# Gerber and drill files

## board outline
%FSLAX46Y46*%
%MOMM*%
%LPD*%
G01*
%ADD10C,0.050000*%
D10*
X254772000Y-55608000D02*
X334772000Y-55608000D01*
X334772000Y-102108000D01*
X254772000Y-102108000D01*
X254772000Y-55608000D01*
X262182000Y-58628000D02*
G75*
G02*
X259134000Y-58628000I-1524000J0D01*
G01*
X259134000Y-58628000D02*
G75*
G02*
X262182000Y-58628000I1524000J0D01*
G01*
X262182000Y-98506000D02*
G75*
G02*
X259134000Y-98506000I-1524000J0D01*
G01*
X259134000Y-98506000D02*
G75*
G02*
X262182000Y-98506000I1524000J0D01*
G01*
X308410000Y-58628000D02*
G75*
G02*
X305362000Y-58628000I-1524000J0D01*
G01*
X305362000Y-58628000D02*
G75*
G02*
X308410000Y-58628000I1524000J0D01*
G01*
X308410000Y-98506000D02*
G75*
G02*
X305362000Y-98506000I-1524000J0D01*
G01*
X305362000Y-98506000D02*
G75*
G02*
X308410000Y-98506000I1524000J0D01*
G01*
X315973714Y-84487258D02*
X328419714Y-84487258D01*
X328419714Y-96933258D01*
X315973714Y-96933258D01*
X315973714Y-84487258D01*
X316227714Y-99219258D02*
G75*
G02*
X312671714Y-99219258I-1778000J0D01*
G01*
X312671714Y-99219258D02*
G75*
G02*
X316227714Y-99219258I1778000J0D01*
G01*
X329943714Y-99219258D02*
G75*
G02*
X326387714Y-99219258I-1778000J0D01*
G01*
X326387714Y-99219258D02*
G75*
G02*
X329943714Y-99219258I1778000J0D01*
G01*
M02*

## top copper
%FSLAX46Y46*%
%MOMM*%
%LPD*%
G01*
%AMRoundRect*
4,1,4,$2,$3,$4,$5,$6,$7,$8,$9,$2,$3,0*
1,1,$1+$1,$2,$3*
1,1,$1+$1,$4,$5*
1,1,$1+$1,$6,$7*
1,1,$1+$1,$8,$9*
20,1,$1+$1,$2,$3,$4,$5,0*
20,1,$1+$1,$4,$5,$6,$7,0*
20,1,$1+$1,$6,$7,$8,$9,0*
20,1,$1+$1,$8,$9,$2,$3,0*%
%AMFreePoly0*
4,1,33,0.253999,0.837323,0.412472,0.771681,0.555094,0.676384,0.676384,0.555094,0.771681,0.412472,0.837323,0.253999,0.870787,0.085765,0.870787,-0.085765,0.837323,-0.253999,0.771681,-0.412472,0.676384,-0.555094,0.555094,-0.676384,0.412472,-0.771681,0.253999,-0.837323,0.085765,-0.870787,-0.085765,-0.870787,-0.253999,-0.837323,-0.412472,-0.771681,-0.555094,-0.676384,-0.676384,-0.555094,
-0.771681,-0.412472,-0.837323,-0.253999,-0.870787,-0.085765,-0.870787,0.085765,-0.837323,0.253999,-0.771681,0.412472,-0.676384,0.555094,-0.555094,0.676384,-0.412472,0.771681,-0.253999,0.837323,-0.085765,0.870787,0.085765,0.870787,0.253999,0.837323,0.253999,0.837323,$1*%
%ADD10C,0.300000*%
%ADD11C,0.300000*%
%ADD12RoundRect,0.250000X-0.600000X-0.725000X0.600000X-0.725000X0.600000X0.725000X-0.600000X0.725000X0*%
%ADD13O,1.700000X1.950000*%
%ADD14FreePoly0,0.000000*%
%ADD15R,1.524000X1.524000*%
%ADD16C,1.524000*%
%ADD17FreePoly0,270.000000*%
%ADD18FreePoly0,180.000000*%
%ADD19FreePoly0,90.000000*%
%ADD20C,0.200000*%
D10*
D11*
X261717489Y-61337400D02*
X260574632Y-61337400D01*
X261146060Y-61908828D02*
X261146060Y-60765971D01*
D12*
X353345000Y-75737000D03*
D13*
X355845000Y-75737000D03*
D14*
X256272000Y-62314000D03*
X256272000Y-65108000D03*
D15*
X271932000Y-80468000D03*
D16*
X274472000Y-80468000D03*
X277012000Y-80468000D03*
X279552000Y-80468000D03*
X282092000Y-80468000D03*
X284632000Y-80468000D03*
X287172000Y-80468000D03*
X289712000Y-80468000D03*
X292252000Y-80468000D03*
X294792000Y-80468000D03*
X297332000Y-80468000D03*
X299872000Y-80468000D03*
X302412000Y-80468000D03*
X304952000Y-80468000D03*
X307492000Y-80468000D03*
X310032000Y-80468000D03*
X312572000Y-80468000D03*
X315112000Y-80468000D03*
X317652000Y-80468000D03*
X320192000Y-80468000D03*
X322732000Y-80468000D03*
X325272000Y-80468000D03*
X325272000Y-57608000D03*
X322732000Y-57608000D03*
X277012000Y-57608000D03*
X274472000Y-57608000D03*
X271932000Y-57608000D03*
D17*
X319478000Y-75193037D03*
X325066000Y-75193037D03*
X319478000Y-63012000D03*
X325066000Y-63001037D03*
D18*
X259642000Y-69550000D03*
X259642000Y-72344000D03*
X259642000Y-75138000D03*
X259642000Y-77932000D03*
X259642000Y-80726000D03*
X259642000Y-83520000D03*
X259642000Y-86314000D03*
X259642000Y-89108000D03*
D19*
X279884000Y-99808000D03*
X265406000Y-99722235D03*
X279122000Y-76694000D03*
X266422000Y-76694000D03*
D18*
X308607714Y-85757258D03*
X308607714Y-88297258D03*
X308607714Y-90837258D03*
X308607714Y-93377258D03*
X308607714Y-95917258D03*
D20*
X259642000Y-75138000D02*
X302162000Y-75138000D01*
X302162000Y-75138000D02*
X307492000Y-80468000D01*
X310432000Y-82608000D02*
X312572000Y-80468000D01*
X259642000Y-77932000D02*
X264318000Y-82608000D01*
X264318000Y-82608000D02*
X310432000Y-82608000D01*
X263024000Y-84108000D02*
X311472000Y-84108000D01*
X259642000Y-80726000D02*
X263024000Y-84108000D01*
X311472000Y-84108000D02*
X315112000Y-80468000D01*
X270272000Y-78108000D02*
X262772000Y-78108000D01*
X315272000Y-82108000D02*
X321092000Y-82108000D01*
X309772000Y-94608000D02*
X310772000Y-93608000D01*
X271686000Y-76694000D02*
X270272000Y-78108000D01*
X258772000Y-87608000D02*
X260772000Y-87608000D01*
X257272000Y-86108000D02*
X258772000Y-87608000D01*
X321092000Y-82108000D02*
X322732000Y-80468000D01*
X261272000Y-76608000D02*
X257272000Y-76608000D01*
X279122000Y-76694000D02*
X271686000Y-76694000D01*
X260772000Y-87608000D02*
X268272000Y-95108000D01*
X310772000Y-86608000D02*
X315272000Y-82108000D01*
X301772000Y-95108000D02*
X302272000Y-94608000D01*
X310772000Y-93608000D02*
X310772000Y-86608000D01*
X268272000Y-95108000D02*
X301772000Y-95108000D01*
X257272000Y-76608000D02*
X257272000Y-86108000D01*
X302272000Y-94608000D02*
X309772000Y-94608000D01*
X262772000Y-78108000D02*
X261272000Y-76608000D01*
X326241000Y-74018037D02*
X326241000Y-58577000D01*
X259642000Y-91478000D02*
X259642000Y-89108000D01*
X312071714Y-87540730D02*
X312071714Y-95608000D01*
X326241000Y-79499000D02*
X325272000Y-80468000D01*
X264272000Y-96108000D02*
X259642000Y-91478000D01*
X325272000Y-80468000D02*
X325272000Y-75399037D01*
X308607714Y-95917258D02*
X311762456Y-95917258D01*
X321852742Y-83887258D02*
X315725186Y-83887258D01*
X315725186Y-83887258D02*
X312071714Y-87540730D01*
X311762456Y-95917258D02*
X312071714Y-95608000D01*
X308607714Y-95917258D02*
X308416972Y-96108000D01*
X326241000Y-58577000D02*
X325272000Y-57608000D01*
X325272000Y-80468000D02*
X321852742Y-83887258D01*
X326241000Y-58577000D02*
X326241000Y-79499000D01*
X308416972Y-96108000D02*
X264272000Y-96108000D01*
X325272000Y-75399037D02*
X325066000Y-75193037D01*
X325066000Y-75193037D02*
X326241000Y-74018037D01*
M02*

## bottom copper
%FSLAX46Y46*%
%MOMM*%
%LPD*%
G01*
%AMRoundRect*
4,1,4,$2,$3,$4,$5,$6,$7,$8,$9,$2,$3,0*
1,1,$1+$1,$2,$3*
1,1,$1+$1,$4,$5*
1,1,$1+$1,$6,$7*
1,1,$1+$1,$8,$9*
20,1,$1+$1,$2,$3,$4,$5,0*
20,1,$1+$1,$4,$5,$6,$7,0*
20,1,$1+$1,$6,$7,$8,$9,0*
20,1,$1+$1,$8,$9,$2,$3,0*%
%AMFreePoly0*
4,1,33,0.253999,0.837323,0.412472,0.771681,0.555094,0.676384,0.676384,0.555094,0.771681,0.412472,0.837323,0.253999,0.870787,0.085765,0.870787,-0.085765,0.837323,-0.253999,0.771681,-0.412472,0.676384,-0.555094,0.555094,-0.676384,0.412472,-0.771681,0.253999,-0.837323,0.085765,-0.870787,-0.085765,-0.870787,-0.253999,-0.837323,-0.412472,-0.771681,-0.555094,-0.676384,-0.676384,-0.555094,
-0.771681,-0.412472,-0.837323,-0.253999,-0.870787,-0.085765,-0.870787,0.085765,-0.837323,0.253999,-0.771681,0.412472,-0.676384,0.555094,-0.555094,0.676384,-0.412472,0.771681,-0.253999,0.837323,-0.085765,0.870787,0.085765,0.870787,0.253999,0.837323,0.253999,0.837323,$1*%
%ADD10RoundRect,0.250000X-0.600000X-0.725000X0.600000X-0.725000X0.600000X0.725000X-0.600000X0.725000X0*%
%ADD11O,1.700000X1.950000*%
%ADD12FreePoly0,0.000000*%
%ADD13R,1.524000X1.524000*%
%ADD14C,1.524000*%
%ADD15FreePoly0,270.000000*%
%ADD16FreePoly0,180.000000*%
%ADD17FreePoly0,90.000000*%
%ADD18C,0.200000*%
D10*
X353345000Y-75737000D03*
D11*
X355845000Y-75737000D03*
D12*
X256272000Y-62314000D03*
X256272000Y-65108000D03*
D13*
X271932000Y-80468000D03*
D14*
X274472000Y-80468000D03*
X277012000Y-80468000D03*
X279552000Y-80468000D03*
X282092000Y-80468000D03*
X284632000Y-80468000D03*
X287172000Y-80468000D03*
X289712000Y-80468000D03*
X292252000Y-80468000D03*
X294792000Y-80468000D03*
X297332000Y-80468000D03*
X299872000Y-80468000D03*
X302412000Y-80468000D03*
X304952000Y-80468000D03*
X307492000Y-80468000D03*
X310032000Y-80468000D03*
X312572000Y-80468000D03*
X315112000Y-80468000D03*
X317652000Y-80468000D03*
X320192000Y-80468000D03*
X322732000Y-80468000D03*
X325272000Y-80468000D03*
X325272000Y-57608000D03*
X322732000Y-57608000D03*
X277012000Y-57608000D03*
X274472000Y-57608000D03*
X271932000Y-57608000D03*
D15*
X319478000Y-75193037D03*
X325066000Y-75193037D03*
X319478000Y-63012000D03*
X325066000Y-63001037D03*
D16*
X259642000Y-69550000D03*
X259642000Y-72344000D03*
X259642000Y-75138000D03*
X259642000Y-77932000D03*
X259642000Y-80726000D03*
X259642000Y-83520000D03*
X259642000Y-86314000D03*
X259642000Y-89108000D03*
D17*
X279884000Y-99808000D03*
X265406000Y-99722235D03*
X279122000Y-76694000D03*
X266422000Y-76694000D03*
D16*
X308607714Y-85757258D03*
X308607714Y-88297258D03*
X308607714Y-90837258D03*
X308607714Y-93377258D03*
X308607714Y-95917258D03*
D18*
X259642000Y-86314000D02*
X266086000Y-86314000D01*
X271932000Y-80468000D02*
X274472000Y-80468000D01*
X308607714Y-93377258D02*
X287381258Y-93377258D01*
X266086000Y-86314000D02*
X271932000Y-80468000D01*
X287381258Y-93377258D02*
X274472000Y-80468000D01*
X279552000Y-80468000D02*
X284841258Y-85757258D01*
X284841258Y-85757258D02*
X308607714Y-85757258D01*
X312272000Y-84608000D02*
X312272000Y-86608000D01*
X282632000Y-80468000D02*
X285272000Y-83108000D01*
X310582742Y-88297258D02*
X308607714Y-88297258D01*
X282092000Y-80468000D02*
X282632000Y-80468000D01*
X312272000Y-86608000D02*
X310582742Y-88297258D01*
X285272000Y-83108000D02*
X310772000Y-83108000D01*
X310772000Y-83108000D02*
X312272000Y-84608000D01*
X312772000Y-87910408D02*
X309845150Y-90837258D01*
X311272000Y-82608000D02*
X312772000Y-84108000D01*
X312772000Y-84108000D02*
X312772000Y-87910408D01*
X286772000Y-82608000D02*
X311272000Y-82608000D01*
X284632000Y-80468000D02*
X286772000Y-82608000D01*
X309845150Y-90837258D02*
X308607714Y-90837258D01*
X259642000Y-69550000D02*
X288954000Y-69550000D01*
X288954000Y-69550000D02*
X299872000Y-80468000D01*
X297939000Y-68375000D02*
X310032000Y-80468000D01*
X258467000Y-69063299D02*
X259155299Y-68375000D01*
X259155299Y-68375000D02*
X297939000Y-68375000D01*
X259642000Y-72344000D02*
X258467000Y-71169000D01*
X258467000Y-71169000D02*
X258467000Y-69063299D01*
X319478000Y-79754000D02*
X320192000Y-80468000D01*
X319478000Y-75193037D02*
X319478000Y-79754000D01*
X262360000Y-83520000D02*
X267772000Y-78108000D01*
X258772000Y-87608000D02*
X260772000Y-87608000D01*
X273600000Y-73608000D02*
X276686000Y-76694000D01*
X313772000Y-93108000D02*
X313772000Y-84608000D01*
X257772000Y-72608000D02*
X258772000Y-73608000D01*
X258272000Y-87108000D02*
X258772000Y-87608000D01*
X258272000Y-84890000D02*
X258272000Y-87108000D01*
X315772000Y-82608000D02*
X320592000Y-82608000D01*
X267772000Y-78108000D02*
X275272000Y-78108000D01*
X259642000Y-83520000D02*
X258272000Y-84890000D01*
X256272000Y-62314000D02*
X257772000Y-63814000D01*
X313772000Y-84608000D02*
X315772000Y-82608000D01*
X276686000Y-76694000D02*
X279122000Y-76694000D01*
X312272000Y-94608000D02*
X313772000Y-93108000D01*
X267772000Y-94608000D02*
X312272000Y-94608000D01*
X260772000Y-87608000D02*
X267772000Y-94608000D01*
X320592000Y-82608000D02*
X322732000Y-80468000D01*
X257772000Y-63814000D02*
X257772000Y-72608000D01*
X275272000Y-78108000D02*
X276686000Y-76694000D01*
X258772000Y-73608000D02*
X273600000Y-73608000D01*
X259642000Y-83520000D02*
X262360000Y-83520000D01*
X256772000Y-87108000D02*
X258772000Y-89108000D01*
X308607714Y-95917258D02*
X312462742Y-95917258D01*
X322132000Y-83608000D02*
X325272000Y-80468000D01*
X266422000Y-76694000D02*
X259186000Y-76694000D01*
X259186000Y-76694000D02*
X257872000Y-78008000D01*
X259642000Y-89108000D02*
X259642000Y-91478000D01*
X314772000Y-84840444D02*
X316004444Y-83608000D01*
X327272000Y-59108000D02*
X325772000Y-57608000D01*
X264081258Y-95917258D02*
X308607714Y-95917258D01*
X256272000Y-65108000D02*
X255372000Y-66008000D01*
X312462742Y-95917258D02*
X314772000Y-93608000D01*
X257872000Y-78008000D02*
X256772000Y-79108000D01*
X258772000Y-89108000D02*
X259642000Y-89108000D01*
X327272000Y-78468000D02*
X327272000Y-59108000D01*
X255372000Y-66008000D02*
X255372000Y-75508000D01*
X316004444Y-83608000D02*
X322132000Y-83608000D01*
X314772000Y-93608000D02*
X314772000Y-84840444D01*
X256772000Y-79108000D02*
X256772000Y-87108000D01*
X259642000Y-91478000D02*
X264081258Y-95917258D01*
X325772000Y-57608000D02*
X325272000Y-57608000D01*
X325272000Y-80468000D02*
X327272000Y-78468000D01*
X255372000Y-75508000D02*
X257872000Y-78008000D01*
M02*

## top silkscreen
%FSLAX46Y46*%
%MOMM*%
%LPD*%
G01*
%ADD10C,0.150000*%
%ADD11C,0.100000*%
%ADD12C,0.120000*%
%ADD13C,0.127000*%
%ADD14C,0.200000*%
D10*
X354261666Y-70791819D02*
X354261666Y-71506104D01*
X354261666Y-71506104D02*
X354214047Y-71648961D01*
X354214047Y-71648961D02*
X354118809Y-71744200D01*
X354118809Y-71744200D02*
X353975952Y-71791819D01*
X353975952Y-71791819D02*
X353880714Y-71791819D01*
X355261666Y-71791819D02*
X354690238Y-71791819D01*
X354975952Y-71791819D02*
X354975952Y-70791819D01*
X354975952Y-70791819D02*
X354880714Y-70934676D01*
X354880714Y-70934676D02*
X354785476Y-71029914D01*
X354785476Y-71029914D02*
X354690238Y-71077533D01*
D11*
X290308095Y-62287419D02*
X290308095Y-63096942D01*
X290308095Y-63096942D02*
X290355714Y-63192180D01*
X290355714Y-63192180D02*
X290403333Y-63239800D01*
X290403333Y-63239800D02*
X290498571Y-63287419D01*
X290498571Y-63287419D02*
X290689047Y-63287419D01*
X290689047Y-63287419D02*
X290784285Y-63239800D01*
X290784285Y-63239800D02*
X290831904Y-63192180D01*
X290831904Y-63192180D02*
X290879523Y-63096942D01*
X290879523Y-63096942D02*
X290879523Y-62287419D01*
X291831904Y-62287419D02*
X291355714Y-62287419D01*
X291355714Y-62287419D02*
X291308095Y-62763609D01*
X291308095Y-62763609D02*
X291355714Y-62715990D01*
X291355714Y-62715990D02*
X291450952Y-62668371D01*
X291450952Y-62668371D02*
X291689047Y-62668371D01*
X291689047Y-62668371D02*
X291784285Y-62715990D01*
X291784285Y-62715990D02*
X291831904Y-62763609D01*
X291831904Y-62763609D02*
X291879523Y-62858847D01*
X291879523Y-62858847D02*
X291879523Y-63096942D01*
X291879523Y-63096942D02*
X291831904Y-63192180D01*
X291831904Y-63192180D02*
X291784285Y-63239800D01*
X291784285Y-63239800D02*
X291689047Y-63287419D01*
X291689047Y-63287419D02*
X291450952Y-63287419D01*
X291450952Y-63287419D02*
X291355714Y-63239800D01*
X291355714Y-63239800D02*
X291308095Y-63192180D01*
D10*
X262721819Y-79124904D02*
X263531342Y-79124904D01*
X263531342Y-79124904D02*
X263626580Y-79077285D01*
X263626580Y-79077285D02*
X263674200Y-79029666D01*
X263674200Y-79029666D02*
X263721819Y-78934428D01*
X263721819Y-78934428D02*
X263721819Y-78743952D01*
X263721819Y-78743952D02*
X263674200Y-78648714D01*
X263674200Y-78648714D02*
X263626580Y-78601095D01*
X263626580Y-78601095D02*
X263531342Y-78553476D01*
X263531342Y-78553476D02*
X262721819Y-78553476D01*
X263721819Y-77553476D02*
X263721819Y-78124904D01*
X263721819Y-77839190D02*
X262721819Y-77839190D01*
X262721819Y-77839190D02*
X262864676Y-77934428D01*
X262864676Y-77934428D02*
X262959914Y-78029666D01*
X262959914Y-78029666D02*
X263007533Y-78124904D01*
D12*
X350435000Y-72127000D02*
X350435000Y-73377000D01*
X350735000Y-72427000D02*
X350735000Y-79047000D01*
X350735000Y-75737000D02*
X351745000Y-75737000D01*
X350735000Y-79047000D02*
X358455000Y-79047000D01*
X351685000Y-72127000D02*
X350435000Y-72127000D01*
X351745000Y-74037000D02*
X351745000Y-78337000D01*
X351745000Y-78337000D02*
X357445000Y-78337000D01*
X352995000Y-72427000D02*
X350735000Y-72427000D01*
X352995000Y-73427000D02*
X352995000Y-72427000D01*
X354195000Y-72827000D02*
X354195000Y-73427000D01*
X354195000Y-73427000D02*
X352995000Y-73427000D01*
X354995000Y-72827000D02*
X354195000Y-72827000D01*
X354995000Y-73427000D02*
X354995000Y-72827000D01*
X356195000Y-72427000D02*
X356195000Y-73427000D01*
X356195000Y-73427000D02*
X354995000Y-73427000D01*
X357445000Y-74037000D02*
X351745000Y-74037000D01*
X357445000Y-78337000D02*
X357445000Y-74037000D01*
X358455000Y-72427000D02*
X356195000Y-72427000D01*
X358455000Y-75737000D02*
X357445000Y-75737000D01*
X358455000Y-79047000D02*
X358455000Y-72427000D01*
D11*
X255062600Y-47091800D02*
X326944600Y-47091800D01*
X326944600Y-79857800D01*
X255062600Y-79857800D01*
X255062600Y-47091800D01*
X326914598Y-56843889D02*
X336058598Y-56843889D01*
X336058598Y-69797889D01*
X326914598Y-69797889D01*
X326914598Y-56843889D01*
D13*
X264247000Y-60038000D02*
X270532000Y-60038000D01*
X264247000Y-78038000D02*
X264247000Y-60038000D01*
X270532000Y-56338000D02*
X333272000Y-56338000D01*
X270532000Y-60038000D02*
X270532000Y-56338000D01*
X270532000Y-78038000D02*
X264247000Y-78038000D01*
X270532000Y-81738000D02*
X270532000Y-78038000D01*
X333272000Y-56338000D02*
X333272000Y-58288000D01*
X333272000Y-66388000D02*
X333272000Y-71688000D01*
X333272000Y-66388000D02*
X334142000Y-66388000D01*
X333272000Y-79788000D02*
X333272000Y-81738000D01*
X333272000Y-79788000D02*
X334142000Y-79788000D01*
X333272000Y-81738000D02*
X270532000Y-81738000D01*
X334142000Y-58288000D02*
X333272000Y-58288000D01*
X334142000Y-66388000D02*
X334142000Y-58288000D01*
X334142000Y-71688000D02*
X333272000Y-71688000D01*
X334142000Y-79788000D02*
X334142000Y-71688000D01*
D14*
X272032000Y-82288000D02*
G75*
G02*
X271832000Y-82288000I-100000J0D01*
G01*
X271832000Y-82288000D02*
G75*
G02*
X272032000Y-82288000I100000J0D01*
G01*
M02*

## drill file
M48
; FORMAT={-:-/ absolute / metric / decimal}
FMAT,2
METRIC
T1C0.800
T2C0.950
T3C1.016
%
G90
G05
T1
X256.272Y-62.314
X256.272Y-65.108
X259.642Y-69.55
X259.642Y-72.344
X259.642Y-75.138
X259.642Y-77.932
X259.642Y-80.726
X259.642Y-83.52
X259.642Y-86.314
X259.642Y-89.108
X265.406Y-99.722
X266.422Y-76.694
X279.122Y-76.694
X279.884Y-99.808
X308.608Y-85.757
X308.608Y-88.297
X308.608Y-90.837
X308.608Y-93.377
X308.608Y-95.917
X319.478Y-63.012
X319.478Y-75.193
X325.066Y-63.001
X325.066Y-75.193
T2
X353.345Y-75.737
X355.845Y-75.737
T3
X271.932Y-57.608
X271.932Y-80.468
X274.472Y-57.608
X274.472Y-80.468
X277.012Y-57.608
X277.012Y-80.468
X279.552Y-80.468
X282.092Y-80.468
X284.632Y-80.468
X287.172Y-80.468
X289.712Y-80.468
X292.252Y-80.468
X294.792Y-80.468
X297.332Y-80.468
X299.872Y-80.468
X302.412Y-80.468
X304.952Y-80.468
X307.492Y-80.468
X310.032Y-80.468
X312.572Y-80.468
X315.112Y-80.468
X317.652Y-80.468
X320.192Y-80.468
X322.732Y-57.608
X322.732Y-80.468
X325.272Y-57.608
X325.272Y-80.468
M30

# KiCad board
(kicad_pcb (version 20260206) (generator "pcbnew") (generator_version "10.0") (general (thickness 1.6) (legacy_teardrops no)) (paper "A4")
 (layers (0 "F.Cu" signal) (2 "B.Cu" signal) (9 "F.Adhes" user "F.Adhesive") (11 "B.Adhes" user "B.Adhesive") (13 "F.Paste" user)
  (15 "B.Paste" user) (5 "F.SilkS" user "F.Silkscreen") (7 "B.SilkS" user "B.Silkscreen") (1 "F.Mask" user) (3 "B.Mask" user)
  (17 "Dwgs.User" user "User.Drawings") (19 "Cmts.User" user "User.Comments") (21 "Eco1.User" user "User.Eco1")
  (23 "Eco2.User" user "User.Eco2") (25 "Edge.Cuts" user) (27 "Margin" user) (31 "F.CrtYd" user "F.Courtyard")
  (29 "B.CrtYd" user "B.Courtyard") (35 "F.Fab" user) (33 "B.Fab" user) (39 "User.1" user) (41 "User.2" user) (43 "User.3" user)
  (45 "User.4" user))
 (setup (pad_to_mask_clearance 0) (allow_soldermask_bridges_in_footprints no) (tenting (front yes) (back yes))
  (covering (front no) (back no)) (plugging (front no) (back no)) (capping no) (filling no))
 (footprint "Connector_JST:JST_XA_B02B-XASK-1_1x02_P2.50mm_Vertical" (layer "F.Cu") (at 353.345 75.737)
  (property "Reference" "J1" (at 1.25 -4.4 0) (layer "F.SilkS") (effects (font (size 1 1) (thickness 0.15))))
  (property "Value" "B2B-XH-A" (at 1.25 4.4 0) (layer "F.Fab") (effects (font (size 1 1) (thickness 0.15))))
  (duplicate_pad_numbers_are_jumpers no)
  (fp_line (start -2.91 -3.61) (end -2.91 -2.36) (stroke (width 0.12) (type solid)) (layer "F.SilkS"))
  (fp_line (start -2.61 -3.31) (end -2.61 3.31) (stroke (width 0.12) (type solid)) (layer "F.SilkS"))
  (fp_line (start -2.61 0) (end -1.6 0) (stroke (width 0.12) (type solid)) (layer "F.SilkS"))
  (fp_line (start -2.61 3.31) (end 5.11 3.31) (stroke (width 0.12) (type solid)) (layer "F.SilkS"))
  (fp_line (start -1.66 -3.61) (end -2.91 -3.61) (stroke (width 0.12) (type solid)) (layer "F.SilkS"))
  (fp_line (start -1.6 -1.7) (end -1.6 2.6) (stroke (width 0.12) (type solid)) (layer "F.SilkS"))
  (fp_line (start -1.6 2.6) (end 4.1 2.6) (stroke (width 0.12) (type solid)) (layer "F.SilkS"))
  (fp_line (start -0.35 -3.31) (end -2.61 -3.31) (stroke (width 0.12) (type solid)) (layer "F.SilkS"))
  (fp_line (start -0.35 -2.31) (end -0.35 -3.31) (stroke (width 0.12) (type solid)) (layer "F.SilkS"))
  (fp_line (start 0.85 -2.91) (end 0.85 -2.31) (stroke (width 0.12) (type solid)) (layer "F.SilkS"))
  (fp_line (start 0.85 -2.31) (end -0.35 -2.31) (stroke (width 0.12) (type solid)) (layer "F.SilkS"))
  (fp_line (start 1.65 -2.91) (end 0.85 -2.91) (stroke (width 0.12) (type solid)) (layer "F.SilkS"))
  (fp_line (start 1.65 -2.31) (end 1.65 -2.91) (stroke (width 0.12) (type solid)) (layer "F.SilkS"))
  (fp_line (start 2.85 -3.31) (end 2.85 -2.31) (stroke (width 0.12) (type solid)) (layer "F.SilkS"))
  (fp_line (start 2.85 -2.31) (end 1.65 -2.31) (stroke (width 0.12) (type solid)) (layer "F.SilkS"))
  (fp_line (start 4.1 -1.7) (end -1.6 -1.7) (stroke (width 0.12) (type solid)) (layer "F.SilkS"))
  (fp_line (start 4.1 2.6) (end 4.1 -1.7) (stroke (width 0.12) (type solid)) (layer "F.SilkS"))
  (fp_line (start 5.11 -3.31) (end 2.85 -3.31) (stroke (width 0.12) (type solid)) (layer "F.SilkS"))
  (fp_line (start 5.11 0) (end 4.1 0) (stroke (width 0.12) (type solid)) (layer "F.SilkS"))
  (fp_line (start 5.11 3.31) (end 5.11 -3.31) (stroke (width 0.12) (type solid)) (layer "F.SilkS"))
  (pad "1" thru_hole roundrect (at 0 0) (size 1.7 1.95) (drill 0.95) (layers "*.Cu" "*.Mask") (remove_unused_layers no)
   (roundrect_rratio 0.147059) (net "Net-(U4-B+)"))
  (pad "2" thru_hole oval (at 2.5 0) (size 1.7 1.95) (drill 0.95) (layers "*.Cu" "*.Mask") (remove_unused_layers no) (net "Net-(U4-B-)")))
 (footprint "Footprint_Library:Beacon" (layer "F.Cu") (at 291.07 63.33)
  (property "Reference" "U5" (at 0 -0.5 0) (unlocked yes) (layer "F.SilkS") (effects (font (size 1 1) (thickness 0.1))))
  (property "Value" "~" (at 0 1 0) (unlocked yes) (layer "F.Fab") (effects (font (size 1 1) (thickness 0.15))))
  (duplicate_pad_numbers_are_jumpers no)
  (fp_rect (start -36.0074 -16.2382) (end 35.8746 16.5278) (stroke (width 0.1) (type default)) (fill no) (layer "F.SilkS"))
  (fp_rect (start 35.844598 -6.486111) (end 44.988598 6.467889) (stroke (width 0.1) (type default)) (fill no) (layer "F.SilkS"))
  (pad "1" thru_hole custom (at -34.798 -1.016) (size 1.75 1.75) (drill 0.8) (layers "*.Cu" "*.Mask") (remove_unused_layers no)
   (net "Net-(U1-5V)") (thermal_bridge_angle 90) (options (clearance outline) (anchor circle)) (primitives))
  (pad "2" thru_hole custom (at -34.798 1.778) (size 1.75 1.75) (drill 0.8) (layers "*.Cu" "*.Mask") (remove_unused_layers no)
   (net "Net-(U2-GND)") (thermal_bridge_angle 90) (options (clearance outline) (anchor circle)) (primitives)))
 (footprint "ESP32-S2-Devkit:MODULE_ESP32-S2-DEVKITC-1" (layer "F.Cu") (at 301.902 69.038 90)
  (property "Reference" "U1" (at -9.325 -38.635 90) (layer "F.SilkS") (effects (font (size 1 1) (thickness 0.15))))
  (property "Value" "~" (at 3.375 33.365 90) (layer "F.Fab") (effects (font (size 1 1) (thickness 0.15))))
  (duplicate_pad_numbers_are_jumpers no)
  (fp_line (start 9 -37.655) (end 9 -31.37) (stroke (width 0.127) (type solid)) (layer "F.SilkS"))
  (fp_line (start -9 -37.655) (end 9 -37.655) (stroke (width 0.127) (type solid)) (layer "F.SilkS"))
  (fp_line (start 12.7 -31.37) (end 12.7 31.37) (stroke (width 0.127) (type solid)) (layer "F.SilkS"))
  (fp_line (start 9 -31.37) (end 12.7 -31.37) (stroke (width 0.127) (type solid)) (layer "F.SilkS"))
  (fp_line (start -9 -31.37) (end -9 -37.655) (stroke (width 0.127) (type solid)) (layer "F.SilkS"))
  (fp_line (start -12.7 -31.37) (end -9 -31.37) (stroke (width 0.127) (type solid)) (layer "F.SilkS"))
  (fp_line (start 12.7 31.37) (end 10.75 31.37) (stroke (width 0.127) (type solid)) (layer "F.SilkS"))
  (fp_line (start 2.65 31.37) (end -2.65 31.37) (stroke (width 0.127) (type solid)) (layer "F.SilkS"))
  (fp_line (start 2.65 31.37) (end 2.65 32.24) (stroke (width 0.127) (type solid)) (layer "F.SilkS"))
  (fp_line (start -10.75 31.37) (end -12.7 31.37) (stroke (width 0.127) (type solid)) (layer "F.SilkS"))
  (fp_line (start -10.75 31.37) (end -10.75 32.24) (stroke (width 0.127) (type solid)) (layer "F.SilkS"))
  (fp_line (start -12.7 31.37) (end -12.7 -31.37) (stroke (width 0.127) (type solid)) (layer "F.SilkS"))
  (fp_line (start 10.75 32.24) (end 10.75 31.37) (stroke (width 0.127) (type solid)) (layer "F.SilkS"))
  (fp_line (start 2.65 32.24) (end 10.75 32.24) (stroke (width 0.127) (type solid)) (layer "F.SilkS"))
  (fp_line (start -2.65 32.24) (end -2.65 31.37) (stroke (width 0.127) (type solid)) (layer "F.SilkS"))
  (fp_line (start -10.75 32.24) (end -2.65 32.24) (stroke (width 0.127) (type solid)) (layer "F.SilkS"))
  (fp_circle (center -13.25 -29.97) (end -13.15 -29.97) (stroke (width 0.2) (type solid)) (fill no) (layer "F.SilkS"))
  (pad "1" thru_hole rect (at -11.43 -29.97 90) (size 1.524 1.524) (drill 1.016) (layers "*.Cu" "*.Mask") (remove_unused_layers no)
   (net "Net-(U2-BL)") (solder_mask_margin 0.102))
  (pad "2" thru_hole circle (at -11.43 -27.43 90) (size 1.524 1.524) (drill 1.016) (layers "*.Cu" "*.Mask") (remove_unused_layers no)
   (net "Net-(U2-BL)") (solder_mask_margin 0.102))
  (pad "3" thru_hole circle (at -11.43 -24.89 90) (size 1.524 1.524) (drill 1.016) (layers "*.Cu" "*.Mask") (remove_unused_layers no)
   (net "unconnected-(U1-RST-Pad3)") (solder_mask_margin 0.102))
  (pad "4" thru_hole circle (at -11.43 -22.35 90) (size 1.524 1.524) (drill 1.016) (layers "*.Cu" "*.Mask") (remove_unused_layers no)
   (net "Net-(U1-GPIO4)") (solder_mask_margin 0.102))
  (pad "5" thru_hole circle (at -11.43 -19.81 90) (size 1.524 1.524) (drill 1.016) (layers "*.Cu" "*.Mask") (remove_unused_layers no)
   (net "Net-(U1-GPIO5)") (solder_mask_margin 0.102))
  (pad "6" thru_hole circle (at -11.43 -17.27 90) (size 1.524 1.524) (drill 1.016) (layers "*.Cu" "*.Mask") (remove_unused_layers no)
   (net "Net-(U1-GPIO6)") (solder_mask_margin 0.102))
  (pad "7" thru_hole circle (at -11.43 -14.73 90) (size 1.524 1.524) (drill 1.016) (layers "*.Cu" "*.Mask") (remove_unused_layers no)
   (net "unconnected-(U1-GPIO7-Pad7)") (solder_mask_margin 0.102))
  (pad "8" thru_hole circle (at -11.43 -12.19 90) (size 1.524 1.524) (drill 1.016) (layers "*.Cu" "*.Mask") (remove_unused_layers no)
   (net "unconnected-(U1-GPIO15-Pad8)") (solder_mask_margin 0.102))
  (pad "9" thru_hole circle (at -11.43 -9.65 90) (size 1.524 1.524) (drill 1.016) (layers "*.Cu" "*.Mask") (remove_unused_layers no)
   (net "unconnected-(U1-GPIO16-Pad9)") (solder_mask_margin 0.102))
  (pad "10" thru_hole circle (at -11.43 -7.11 90) (size 1.524 1.524) (drill 1.016) (layers "*.Cu" "*.Mask") (remove_unused_layers no)
   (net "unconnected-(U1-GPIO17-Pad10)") (solder_mask_margin 0.102))
  (pad "11" thru_hole circle (at -11.43 -4.57 90) (size 1.524 1.524) (drill 1.016) (layers "*.Cu" "*.Mask") (remove_unused_layers no)
   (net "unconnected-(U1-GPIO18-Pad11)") (solder_mask_margin 0.102))
  (pad "12" thru_hole circle (at -11.43 -2.03 90) (size 1.524 1.524) (drill 1.016) (layers "*.Cu" "*.Mask") (remove_unused_layers no)
   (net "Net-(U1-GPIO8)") (solder_mask_margin 0.102))
  (pad "13" thru_hole circle (at -11.43 0.51 90) (size 1.524 1.524) (drill 1.016) (layers "*.Cu" "*.Mask") (remove_unused_layers no)
   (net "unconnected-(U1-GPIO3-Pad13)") (solder_mask_margin 0.102))
  (pad "14" thru_hole circle (at -11.43 3.05 90) (size 1.524 1.524) (drill 1.016) (layers "*.Cu" "*.Mask") (remove_unused_layers no)
   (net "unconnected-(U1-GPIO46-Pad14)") (solder_mask_margin 0.102))
  (pad "15" thru_hole circle (at -11.43 5.59 90) (size 1.524 1.524) (drill 1.016) (layers "*.Cu" "*.Mask") (remove_unused_layers no)
   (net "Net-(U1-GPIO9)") (solder_mask_margin 0.102))
  (pad "16" thru_hole circle (at -11.43 8.13 90) (size 1.524 1.524) (drill 1.016) (layers "*.Cu" "*.Mask") (remove_unused_layers no)
   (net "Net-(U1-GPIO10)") (solder_mask_margin 0.102))
  (pad "17" thru_hole circle (at -11.43 10.67 90) (size 1.524 1.524) (drill 1.016) (layers "*.Cu" "*.Mask") (remove_unused_layers no)
   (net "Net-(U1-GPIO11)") (solder_mask_margin 0.102))
  (pad "18" thru_hole circle (at -11.43 13.21 90) (size 1.524 1.524) (drill 1.016) (layers "*.Cu" "*.Mask") (remove_unused_layers no)
   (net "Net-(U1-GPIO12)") (solder_mask_margin 0.102))
  (pad "19" thru_hole circle (at -11.43 15.75 90) (size 1.524 1.524) (drill 1.016) (layers "*.Cu" "*.Mask") (remove_unused_layers no)
   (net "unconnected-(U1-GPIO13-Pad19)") (solder_mask_margin 0.102))
  (pad "20" thru_hole circle (at -11.43 18.29 90) (size 1.524 1.524) (drill 1.016) (layers "*.Cu" "*.Mask") (remove_unused_layers no)
   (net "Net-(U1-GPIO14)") (solder_mask_margin 0.102))
  (pad "21" thru_hole circle (at -11.43 20.83 90) (size 1.524 1.524) (drill 1.016) (layers "*.Cu" "*.Mask") (remove_unused_layers no)
   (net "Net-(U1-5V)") (solder_mask_margin 0.102))
  (pad "22" thru_hole circle (at -11.43 23.37 90) (size 1.524 1.524) (drill 1.016) (layers "*.Cu" "*.Mask") (remove_unused_layers no)
   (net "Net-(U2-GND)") (solder_mask_margin 0.102))
  (pad "23" thru_hole circle (at 11.43 23.37 90) (size 1.524 1.524) (drill 1.016) (layers "*.Cu" "*.Mask") (remove_unused_layers no)
   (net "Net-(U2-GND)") (solder_mask_margin 0.102))
  (pad "24" thru_hole circle (at 11.43 20.83 90) (size 1.524 1.524) (drill 1.016) (layers "*.Cu" "*.Mask") (remove_unused_layers no)
   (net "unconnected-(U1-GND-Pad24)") (solder_mask_margin 0.102))
  (pad "42" thru_hole circle (at 11.43 -24.89 90) (size 1.524 1.524) (drill 1.016) (layers "*.Cu" "*.Mask") (remove_unused_layers no)
   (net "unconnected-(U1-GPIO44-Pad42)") (solder_mask_margin 0.102))
  (pad "43" thru_hole circle (at 11.43 -27.43 90) (size 1.524 1.524) (drill 1.016) (layers "*.Cu" "*.Mask") (remove_unused_layers no)
   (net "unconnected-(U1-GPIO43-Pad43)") (solder_mask_margin 0.102))
  (pad "44" thru_hole circle (at 11.43 -29.97 90) (size 1.524 1.524) (drill 1.016) (layers "*.Cu" "*.Mask") (remove_unused_layers no)
   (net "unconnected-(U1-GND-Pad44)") (solder_mask_margin 0.102)))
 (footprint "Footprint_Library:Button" (layer "B.Cu") (at 322.272 69.108 -90)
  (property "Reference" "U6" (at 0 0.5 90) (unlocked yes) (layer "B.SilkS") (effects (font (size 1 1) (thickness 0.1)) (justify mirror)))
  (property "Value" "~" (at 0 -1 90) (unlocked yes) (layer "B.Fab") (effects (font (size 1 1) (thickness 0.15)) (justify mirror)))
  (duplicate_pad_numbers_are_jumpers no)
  (pad "1" thru_hole custom (at 6.085037 2.794 270) (size 1.75 1.75) (drill 0.8) (layers "*.Cu" "*.Mask") (remove_unused_layers no)
   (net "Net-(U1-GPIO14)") (thermal_bridge_angle 90) (options (clearance outline) (anchor circle)) (primitives))
  (pad "2" thru_hole custom (at 6.085037 -2.794 270) (size 1.75 1.75) (drill 0.8) (layers "*.Cu" "*.Mask") (remove_unused_layers no)
   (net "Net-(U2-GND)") (thermal_bridge_angle 90) (options (clearance outline) (anchor circle)) (primitives))
  (pad "3" thru_hole custom (at -6.096 2.794 270) (size 1.75 1.75) (drill 0.8) (layers "*.Cu" "*.Mask") (remove_unused_layers no)
   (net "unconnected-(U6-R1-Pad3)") (thermal_bridge_angle 90) (options (clearance outline) (anchor circle)) (primitives))
  (pad "4" thru_hole custom (at -6.106963 -2.794 270) (size 1.75 1.75) (drill 0.8) (layers "*.Cu" "*.Mask") (remove_unused_layers no)
   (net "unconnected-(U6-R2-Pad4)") (thermal_bridge_angle 90) (options (clearance outline) (anchor circle)) (primitives)))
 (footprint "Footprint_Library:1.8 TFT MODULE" (layer "B.Cu") (at 283.772 80.218 180)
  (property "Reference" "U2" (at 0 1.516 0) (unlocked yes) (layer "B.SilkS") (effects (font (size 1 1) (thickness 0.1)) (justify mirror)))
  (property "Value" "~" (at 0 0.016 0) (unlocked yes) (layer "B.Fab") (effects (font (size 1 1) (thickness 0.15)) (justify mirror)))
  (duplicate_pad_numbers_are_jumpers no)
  (fp_circle (center 23.114 21.59) (end 24.638 21.59) (stroke (width 0.05) (type default)) (fill no) (layer "Edge.Cuts"))
  (fp_circle (center 23.114 -18.288) (end 24.638 -18.288) (stroke (width 0.05) (type default)) (fill no) (layer "Edge.Cuts"))
  (fp_circle (center -23.114 21.59) (end -21.59 21.59) (stroke (width 0.05) (type default)) (fill no) (layer "Edge.Cuts"))
  (fp_circle (center -23.114 -18.288) (end -21.59 -18.288) (stroke (width 0.05) (type default)) (fill no) (layer "Edge.Cuts"))
  (pad "1" thru_hole custom (at 24.13 10.668 180) (size 1.75 1.75) (drill 0.8) (layers "*.Cu" "*.Mask") (remove_unused_layers no)
   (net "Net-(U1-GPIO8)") (thermal_bridge_angle 90) (options (clearance outline) (anchor circle)) (primitives))
  (pad "2" thru_hole custom (at 24.13 7.874 180) (size 1.75 1.75) (drill 0.8) (layers "*.Cu" "*.Mask") (remove_unused_layers no)
   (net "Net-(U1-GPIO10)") (thermal_bridge_angle 90) (options (clearance outline) (anchor circle)) (primitives))
  (pad "3" thru_hole custom (at 24.13 5.08 180) (size 1.75 1.75) (drill 0.8) (layers "*.Cu" "*.Mask") (remove_unused_layers no)
   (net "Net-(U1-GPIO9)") (thermal_bridge_angle 90) (options (clearance outline) (anchor circle)) (primitives))
  (pad "4" thru_hole custom (at 24.13 2.286 180) (size 1.75 1.75) (drill 0.8) (layers "*.Cu" "*.Mask") (remove_unused_layers no)
   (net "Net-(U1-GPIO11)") (thermal_bridge_angle 90) (options (clearance outline) (anchor circle)) (primitives))
  (pad "5" thru_hole custom (at 24.13 -0.508 180) (size 1.75 1.75) (drill 0.8) (layers "*.Cu" "*.Mask") (remove_unused_layers no)
   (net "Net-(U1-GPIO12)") (thermal_bridge_angle 90) (options (clearance outline) (anchor circle)) (primitives))
  (pad "6" thru_hole custom (at 24.13 -3.302 180) (size 1.75 1.75) (drill 0.8) (layers "*.Cu" "*.Mask") (remove_unused_layers no)
   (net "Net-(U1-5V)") (thermal_bridge_angle 90) (options (clearance outline) (anchor circle)) (primitives))
  (pad "7" thru_hole custom (at 24.13 -6.096 180) (size 1.75 1.75) (drill 0.8) (layers "*.Cu" "*.Mask") (remove_unused_layers no)
   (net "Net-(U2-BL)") (thermal_bridge_angle 90) (options (clearance outline) (anchor circle)) (primitives))
  (pad "8" thru_hole custom (at 24.13 -8.89 180) (size 1.75 1.75) (drill 0.8) (layers "*.Cu" "*.Mask") (remove_unused_layers no)
   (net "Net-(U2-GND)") (thermal_bridge_angle 90) (options (clearance outline) (anchor circle)) (primitives)))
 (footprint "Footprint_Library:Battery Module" (layer "B.Cu") (at 272.772 87.108 90)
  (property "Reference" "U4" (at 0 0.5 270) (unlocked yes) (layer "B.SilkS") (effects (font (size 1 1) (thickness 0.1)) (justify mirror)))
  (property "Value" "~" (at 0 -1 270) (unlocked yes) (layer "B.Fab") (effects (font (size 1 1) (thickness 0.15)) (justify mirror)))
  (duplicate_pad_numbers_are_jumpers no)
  (pad "1" thru_hole custom (at -12.7 7.112 90) (size 1.75 1.75) (drill 0.8) (layers "*.Cu" "*.Mask") (remove_unused_layers no)
   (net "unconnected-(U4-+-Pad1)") (thermal_bridge_angle 90) (options (clearance outline) (anchor circle)) (primitives))
  (pad "2" thru_hole custom (at -12.614235 -7.366 90) (size 1.75 1.75) (drill 0.8) (layers "*.Cu" "*.Mask") (remove_unused_layers no)
   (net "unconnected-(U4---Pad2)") (thermal_bridge_angle 90) (options (clearance outline) (anchor circle)) (primitives))
  (pad "3" thru_hole custom (at 10.414 6.35 90) (size 1.75 1.75) (drill 0.8) (layers "*.Cu" "*.Mask") (remove_unused_layers no)
   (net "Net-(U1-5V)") (thermal_bridge_angle 90) (options (clearance outline) (anchor circle)) (primitives))
  (pad "6" thru_hole custom (at 10.414 -6.35 90) (size 1.75 1.75) (drill 0.8) (layers "*.Cu" "*.Mask") (remove_unused_layers no)
   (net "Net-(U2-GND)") (thermal_bridge_angle 90) (options (clearance outline) (anchor circle)) (primitives)))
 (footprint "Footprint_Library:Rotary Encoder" (layer "B.Cu") (at 308.607714 85.757258 180)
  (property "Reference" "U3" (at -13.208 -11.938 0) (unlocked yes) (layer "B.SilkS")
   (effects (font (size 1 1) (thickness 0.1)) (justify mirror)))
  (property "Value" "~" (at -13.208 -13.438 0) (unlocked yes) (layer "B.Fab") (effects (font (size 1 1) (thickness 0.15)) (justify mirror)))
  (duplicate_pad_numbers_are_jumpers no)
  (fp_rect (start -19.812 1.27) (end -7.366 -11.176) (stroke (width 0.05) (type default)) (fill no) (layer "Edge.Cuts"))
  (fp_circle (center -5.842 -13.462) (end -4.064 -13.462) (stroke (width 0.05) (type default)) (fill no) (layer "Edge.Cuts"))
  (fp_circle (center -19.558 -13.462) (end -17.78 -13.462) (stroke (width 0.05) (type default)) (fill no) (layer "Edge.Cuts"))
  (pad "1" thru_hole custom (at 0 0 180) (size 1.75 1.75) (drill 0.8) (layers "*.Cu" "*.Mask") (remove_unused_layers no)
   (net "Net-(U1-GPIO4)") (thermal_bridge_angle 90) (options (clearance outline) (anchor circle)) (primitives))
  (pad "2" thru_hole custom (at 0 -2.54 180) (size 1.75 1.75) (drill 0.8) (layers "*.Cu" "*.Mask") (remove_unused_layers no)
   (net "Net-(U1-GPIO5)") (thermal_bridge_angle 90) (options (clearance outline) (anchor circle)) (primitives))
  (pad "3" thru_hole custom (at 0 -5.08 180) (size 1.75 1.75) (drill 0.8) (layers "*.Cu" "*.Mask") (remove_unused_layers no)
   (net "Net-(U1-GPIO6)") (thermal_bridge_angle 90) (options (clearance outline) (anchor circle)) (primitives))
  (pad "4" thru_hole custom (at 0 -7.62 180) (size 1.75 1.75) (drill 0.8) (layers "*.Cu" "*.Mask") (remove_unused_layers no)
   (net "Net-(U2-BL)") (thermal_bridge_angle 90) (options (clearance outline) (anchor circle)) (primitives))
  (pad "5" thru_hole custom (at 0 -10.16 180) (size 1.75 1.75) (drill 0.8) (layers "*.Cu" "*.Mask") (remove_unused_layers no)
   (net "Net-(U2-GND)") (thermal_bridge_angle 90) (options (clearance outline) (anchor circle)) (primitives)))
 (gr_rect (start 254.772 55.608) (end 334.772 102.108) (stroke (width 0.05) (type default)) (fill no) (layer "Edge.Cuts"))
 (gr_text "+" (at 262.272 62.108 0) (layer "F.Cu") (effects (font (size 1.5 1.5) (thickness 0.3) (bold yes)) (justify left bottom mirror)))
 (segment (start 259.642 86.314) (end 266.086 86.314) (width 0.2) (layer "B.Cu") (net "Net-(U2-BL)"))
 (segment (start 271.932 80.468) (end 274.472 80.468) (width 0.2) (layer "B.Cu") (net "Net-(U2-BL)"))
 (segment (start 308.607714 93.377258) (end 287.381258 93.377258) (width 0.2) (layer "B.Cu") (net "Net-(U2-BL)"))
 (segment (start 266.086 86.314) (end 271.932 80.468) (width 0.2) (layer "B.Cu") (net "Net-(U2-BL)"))
 (segment (start 287.381258 93.377258) (end 274.472 80.468) (width 0.2) (layer "B.Cu") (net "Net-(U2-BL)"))
 (segment (start 279.552 80.468) (end 284.841258 85.757258) (width 0.2) (layer "B.Cu") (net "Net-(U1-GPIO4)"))
 (segment (start 284.841258 85.757258) (end 308.607714 85.757258) (width 0.2) (layer "B.Cu") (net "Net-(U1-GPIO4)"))
 (segment (start 312.272 84.608) (end 312.272 86.608) (width 0.2) (layer "B.Cu") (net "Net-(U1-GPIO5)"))
 (segment (start 282.632 80.468) (end 285.272 83.108) (width 0.2) (layer "B.Cu") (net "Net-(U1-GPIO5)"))
 (segment (start 310.582742 88.297258) (end 308.607714 88.297258) (width 0.2) (layer "B.Cu") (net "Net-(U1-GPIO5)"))
 (segment (start 282.092 80.468) (end 282.632 80.468) (width 0.2) (layer "B.Cu") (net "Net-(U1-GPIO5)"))
 (segment (start 312.272 86.608) (end 310.582742 88.297258) (width 0.2) (layer "B.Cu") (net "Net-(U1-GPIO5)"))
 (segment (start 285.272 83.108) (end 310.772 83.108) (width 0.2) (layer "B.Cu") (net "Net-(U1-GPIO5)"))
 (segment (start 310.772 83.108) (end 312.272 84.608) (width 0.2) (layer "B.Cu") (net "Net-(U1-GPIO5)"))
 (segment (start 312.772 87.910408) (end 309.84515 90.837258) (width 0.2) (layer "B.Cu") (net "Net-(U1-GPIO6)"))
 (segment (start 311.272 82.608) (end 312.772 84.108) (width 0.2) (layer "B.Cu") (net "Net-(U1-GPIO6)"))
 (segment (start 312.772 84.108) (end 312.772 87.910408) (width 0.2) (layer "B.Cu") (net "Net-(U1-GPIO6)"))
 (segment (start 286.772 82.608) (end 311.272 82.608) (width 0.2) (layer "B.Cu") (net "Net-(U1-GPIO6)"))
 (segment (start 284.632 80.468) (end 286.772 82.608) (width 0.2) (layer "B.Cu") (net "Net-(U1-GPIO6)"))
 (segment (start 309.84515 90.837258) (end 308.607714 90.837258) (width 0.2) (layer "B.Cu") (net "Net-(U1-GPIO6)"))
 (segment (start 259.642 69.55) (end 288.954 69.55) (width 0.2) (layer "B.Cu") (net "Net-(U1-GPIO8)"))
 (segment (start 288.954 69.55) (end 299.872 80.468) (width 0.2) (layer "B.Cu") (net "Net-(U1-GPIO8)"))
 (segment (start 259.642 75.138) (end 302.162 75.138) (width 0.2) (layer "F.Cu") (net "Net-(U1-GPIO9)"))
 (segment (start 302.162 75.138) (end 307.492 80.468) (width 0.2) (layer "F.Cu") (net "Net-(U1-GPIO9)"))
 (segment (start 297.939 68.375) (end 310.032 80.468) (width 0.2) (layer "B.Cu") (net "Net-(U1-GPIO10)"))
 (segment (start 258.467 69.063299) (end 259.155299 68.375) (width 0.2) (layer "B.Cu") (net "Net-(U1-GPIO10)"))
 (segment (start 259.155299 68.375) (end 297.939 68.375) (width 0.2) (layer "B.Cu") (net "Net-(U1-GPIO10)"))
 (segment (start 259.642 72.344) (end 258.467 71.169) (width 0.2) (layer "B.Cu") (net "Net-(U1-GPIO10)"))
 (segment (start 258.467 71.169) (end 258.467 69.063299) (width 0.2) (layer "B.Cu") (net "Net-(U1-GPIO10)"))
 (segment (start 310.432 82.608) (end 312.572 80.468) (width 0.2) (layer "F.Cu") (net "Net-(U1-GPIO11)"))
 (segment (start 259.642 77.932) (end 264.318 82.608) (width 0.2) (layer "F.Cu") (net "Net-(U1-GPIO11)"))
 (segment (start 264.318 82.608) (end 310.432 82.608) (width 0.2) (layer "F.Cu") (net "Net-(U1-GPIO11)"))
 (segment (start 263.024 84.108) (end 311.472 84.108) (width 0.2) (layer "F.Cu") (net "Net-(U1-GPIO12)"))
 (segment (start 259.642 80.726) (end 263.024 84.108) (width 0.2) (layer "F.Cu") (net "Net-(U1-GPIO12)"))
 (segment (start 311.472 84.108) (end 315.112 80.468) (width 0.2) (layer "F.Cu") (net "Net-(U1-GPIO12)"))
 (segment (start 319.478 79.754) (end 320.192 80.468) (width 0.2) (layer "B.Cu") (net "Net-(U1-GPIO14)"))
 (segment (start 319.478 75.193037) (end 319.478 79.754) (width 0.2) (layer "B.Cu") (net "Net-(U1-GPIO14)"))
 (segment (start 270.272 78.108) (end 262.772 78.108) (width 0.2) (layer "F.Cu") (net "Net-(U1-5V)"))
 (segment (start 315.272 82.108) (end 321.092 82.108) (width 0.2) (layer "F.Cu") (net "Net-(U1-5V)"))
 (segment (start 309.772 94.608) (end 310.772 93.608) (width 0.2) (layer "F.Cu") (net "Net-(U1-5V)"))
 (segment (start 271.686 76.694) (end 270.272 78.108) (width 0.2) (layer "F.Cu") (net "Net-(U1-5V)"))
 (segment (start 258.772 87.608) (end 260.772 87.608) (width 0.2) (layer "F.Cu") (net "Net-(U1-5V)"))
 (segment (start 257.272 86.108) (end 258.772 87.608) (width 0.2) (layer "F.Cu") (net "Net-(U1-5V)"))
 (segment (start 321.092 82.108) (end 322.732 80.468) (width 0.2) (layer "F.Cu") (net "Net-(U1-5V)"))
 (segment (start 261.272 76.608) (end 257.272 76.608) (width 0.2) (layer "F.Cu") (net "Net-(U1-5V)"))
 (segment (start 279.122 76.694) (end 271.686 76.694) (width 0.2) (layer "F.Cu") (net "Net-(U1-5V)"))
 (segment (start 260.772 87.608) (end 268.272 95.108) (width 0.2) (layer "F.Cu") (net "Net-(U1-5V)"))
 (segment (start 310.772 86.608) (end 315.272 82.108) (width 0.2) (layer "F.Cu") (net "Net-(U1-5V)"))
 (segment (start 301.772 95.108) (end 302.272 94.608) (width 0.2) (layer "F.Cu") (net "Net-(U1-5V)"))
 (segment (start 310.772 93.608) (end 310.772 86.608) (width 0.2) (layer "F.Cu") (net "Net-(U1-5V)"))
 (segment (start 268.272 95.108) (end 301.772 95.108) (width 0.2) (layer "F.Cu") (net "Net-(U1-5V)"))
 (segment (start 257.272 76.608) (end 257.272 86.108) (width 0.2) (layer "F.Cu") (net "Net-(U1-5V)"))
 (segment (start 302.272 94.608) (end 309.772 94.608) (width 0.2) (layer "F.Cu") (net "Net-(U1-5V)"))
 (segment (start 262.772 78.108) (end 261.272 76.608) (width 0.2) (layer "F.Cu") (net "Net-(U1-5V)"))
 (segment (start 262.36 83.52) (end 267.772 78.108) (width 0.2) (layer "B.Cu") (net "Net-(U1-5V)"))
 (segment (start 258.772 87.608) (end 260.772 87.608) (width 0.2) (layer "B.Cu") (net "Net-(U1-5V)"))
 (segment (start 273.6 73.608) (end 276.686 76.694) (width 0.2) (layer "B.Cu") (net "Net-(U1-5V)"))
 (segment (start 313.772 93.108) (end 313.772 84.608) (width 0.2) (layer "B.Cu") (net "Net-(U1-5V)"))
 (segment (start 257.772 72.608) (end 258.772 73.608) (width 0.2) (layer "B.Cu") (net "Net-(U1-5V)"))
 (segment (start 258.272 87.108) (end 258.772 87.608) (width 0.2) (layer "B.Cu") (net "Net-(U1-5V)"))
 (segment (start 258.272 84.89) (end 258.272 87.108) (width 0.2) (layer "B.Cu") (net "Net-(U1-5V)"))
 (segment (start 315.772 82.608) (end 320.592 82.608) (width 0.2) (layer "B.Cu") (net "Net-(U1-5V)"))
 (segment (start 267.772 78.108) (end 275.272 78.108) (width 0.2) (layer "B.Cu") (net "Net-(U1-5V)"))
 (segment (start 259.642 83.52) (end 258.272 84.89) (width 0.2) (layer "B.Cu") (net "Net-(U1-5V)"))
 (segment (start 256.272 62.314) (end 257.772 63.814) (width 0.2) (layer "B.Cu") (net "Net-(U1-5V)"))
 (segment (start 313.772 84.608) (end 315.772 82.608) (width 0.2) (layer "B.Cu") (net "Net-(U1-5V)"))
 (segment (start 276.686 76.694) (end 279.122 76.694) (width 0.2) (layer "B.Cu") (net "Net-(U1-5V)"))
 (segment (start 312.272 94.608) (end 313.772 93.108) (width 0.2) (layer "B.Cu") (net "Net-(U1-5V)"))
 (segment (start 267.772 94.608) (end 312.272 94.608) (width 0.2) (layer "B.Cu") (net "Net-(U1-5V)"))
 (segment (start 260.772 87.608) (end 267.772 94.608) (width 0.2) (layer "B.Cu") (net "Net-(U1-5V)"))
 (segment (start 320.592 82.608) (end 322.732 80.468) (width 0.2) (layer "B.Cu") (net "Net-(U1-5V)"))
 (segment (start 257.772 63.814) (end 257.772 72.608) (width 0.2) (layer "B.Cu") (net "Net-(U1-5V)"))
 (segment (start 275.272 78.108) (end 276.686 76.694) (width 0.2) (layer "B.Cu") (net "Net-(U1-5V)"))
 (segment (start 258.772 73.608) (end 273.6 73.608) (width 0.2) (layer "B.Cu") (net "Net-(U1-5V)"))
 (segment (start 259.642 83.52) (end 262.36 83.52) (width 0.2) (layer "B.Cu") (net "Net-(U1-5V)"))
 (segment (start 326.241 74.018037) (end 326.241 58.577) (width 0.2) (layer "F.Cu") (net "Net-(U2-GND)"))
 (segment (start 259.642 91.478) (end 259.642 89.108) (width 0.2) (layer "F.Cu") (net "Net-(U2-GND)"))
 (segment (start 312.071714 87.54073) (end 312.071714 95.608) (width 0.2) (layer "F.Cu") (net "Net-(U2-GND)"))
 (segment (start 326.241 79.499) (end 325.272 80.468) (width 0.2) (layer "F.Cu") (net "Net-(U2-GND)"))
 (segment (start 264.272 96.108) (end 259.642 91.478) (width 0.2) (layer "F.Cu") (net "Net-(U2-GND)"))
 (segment (start 325.272 80.468) (end 325.272 75.399037) (width 0.2) (layer "F.Cu") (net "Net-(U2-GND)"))
 (segment (start 308.607714 95.917258) (end 311.762456 95.917258) (width 0.2) (layer "F.Cu") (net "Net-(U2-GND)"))
 (segment (start 321.852742 83.887258) (end 315.725186 83.887258) (width 0.2) (layer "F.Cu") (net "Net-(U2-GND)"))
 (segment (start 315.725186 83.887258) (end 312.071714 87.54073) (width 0.2) (layer "F.Cu") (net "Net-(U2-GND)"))
 (segment (start 311.762456 95.917258) (end 312.071714 95.608) (width 0.2) (layer "F.Cu") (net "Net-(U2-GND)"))
 (segment (start 308.607714 95.917258) (end 308.416972 96.108) (width 0.2) (layer "F.Cu") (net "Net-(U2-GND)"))
 (segment (start 326.241 58.577) (end 325.272 57.608) (width 0.2) (layer "F.Cu") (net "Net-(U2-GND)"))
 (segment (start 325.272 80.468) (end 321.852742 83.887258) (width 0.2) (layer "F.Cu") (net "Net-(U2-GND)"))
 (segment (start 326.241 58.577) (end 326.241 79.499) (width 0.2) (layer "F.Cu") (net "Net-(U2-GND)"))
 (segment (start 308.416972 96.108) (end 264.272 96.108) (width 0.2) (layer "F.Cu") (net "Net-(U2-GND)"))
 (segment (start 325.272 75.399037) (end 325.066 75.193037) (width 0.2) (layer "F.Cu") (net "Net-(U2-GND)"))
 (segment (start 325.066 75.193037) (end 326.241 74.018037) (width 0.2) (layer "F.Cu") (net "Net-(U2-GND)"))
 (segment (start 256.772 87.108) (end 258.772 89.108) (width 0.2) (layer "B.Cu") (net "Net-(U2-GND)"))
 (segment (start 308.607714 95.917258) (end 312.462742 95.917258) (width 0.2) (layer "B.Cu") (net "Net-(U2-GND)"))
 (segment (start 322.132 83.608) (end 325.272 80.468) (width 0.2) (layer "B.Cu") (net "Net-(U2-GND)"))
 (segment (start 266.422 76.694) (end 259.186 76.694) (width 0.2) (layer "B.Cu") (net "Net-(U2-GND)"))
 (segment (start 259.186 76.694) (end 257.872 78.008) (width 0.2) (layer "B.Cu") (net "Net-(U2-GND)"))
 (segment (start 259.642 89.108) (end 259.642 91.478) (width 0.2) (layer "B.Cu") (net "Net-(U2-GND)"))
 (segment (start 314.772 84.840444) (end 316.004444 83.608) (width 0.2) (layer "B.Cu") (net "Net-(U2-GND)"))
 (segment (start 327.272 59.108) (end 325.772 57.608) (width 0.2) (layer "B.Cu") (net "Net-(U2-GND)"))
 (segment (start 264.081258 95.917258) (end 308.607714 95.917258) (width 0.2) (layer "B.Cu") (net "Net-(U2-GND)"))
 (segment (start 256.272 65.108) (end 255.372 66.008) (width 0.2) (layer "B.Cu") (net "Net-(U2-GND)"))
 (segment (start 312.462742 95.917258) (end 314.772 93.608) (width 0.2) (layer "B.Cu") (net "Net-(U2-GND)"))
 (segment (start 257.872 78.008) (end 256.772 79.108) (width 0.2) (layer "B.Cu") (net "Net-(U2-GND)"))
 (segment (start 258.772 89.108) (end 259.642 89.108) (width 0.2) (layer "B.Cu") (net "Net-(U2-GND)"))
 (segment (start 327.272 78.468) (end 327.272 59.108) (width 0.2) (layer "B.Cu") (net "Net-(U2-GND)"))
 (segment (start 255.372 66.008) (end 255.372 75.508) (width 0.2) (layer "B.Cu") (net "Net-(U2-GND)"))
 (segment (start 316.004444 83.608) (end 322.132 83.608) (width 0.2) (layer "B.Cu") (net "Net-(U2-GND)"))
 (segment (start 314.772 93.608) (end 314.772 84.840444) (width 0.2) (layer "B.Cu") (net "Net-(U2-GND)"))
 (segment (start 256.772 79.108) (end 256.772 87.108) (width 0.2) (layer "B.Cu") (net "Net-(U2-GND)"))
 (segment (start 259.642 91.478) (end 264.081258 95.917258) (width 0.2) (layer "B.Cu") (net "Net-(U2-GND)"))
 (segment (start 325.772 57.608) (end 325.272 57.608) (width 0.2) (layer "B.Cu") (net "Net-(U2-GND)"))
 (segment (start 325.272 80.468) (end 327.272 78.468) (width 0.2) (layer "B.Cu") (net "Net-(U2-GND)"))
 (segment (start 255.372 75.508) (end 257.872 78.008) (width 0.2) (layer "B.Cu") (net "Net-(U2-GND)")))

